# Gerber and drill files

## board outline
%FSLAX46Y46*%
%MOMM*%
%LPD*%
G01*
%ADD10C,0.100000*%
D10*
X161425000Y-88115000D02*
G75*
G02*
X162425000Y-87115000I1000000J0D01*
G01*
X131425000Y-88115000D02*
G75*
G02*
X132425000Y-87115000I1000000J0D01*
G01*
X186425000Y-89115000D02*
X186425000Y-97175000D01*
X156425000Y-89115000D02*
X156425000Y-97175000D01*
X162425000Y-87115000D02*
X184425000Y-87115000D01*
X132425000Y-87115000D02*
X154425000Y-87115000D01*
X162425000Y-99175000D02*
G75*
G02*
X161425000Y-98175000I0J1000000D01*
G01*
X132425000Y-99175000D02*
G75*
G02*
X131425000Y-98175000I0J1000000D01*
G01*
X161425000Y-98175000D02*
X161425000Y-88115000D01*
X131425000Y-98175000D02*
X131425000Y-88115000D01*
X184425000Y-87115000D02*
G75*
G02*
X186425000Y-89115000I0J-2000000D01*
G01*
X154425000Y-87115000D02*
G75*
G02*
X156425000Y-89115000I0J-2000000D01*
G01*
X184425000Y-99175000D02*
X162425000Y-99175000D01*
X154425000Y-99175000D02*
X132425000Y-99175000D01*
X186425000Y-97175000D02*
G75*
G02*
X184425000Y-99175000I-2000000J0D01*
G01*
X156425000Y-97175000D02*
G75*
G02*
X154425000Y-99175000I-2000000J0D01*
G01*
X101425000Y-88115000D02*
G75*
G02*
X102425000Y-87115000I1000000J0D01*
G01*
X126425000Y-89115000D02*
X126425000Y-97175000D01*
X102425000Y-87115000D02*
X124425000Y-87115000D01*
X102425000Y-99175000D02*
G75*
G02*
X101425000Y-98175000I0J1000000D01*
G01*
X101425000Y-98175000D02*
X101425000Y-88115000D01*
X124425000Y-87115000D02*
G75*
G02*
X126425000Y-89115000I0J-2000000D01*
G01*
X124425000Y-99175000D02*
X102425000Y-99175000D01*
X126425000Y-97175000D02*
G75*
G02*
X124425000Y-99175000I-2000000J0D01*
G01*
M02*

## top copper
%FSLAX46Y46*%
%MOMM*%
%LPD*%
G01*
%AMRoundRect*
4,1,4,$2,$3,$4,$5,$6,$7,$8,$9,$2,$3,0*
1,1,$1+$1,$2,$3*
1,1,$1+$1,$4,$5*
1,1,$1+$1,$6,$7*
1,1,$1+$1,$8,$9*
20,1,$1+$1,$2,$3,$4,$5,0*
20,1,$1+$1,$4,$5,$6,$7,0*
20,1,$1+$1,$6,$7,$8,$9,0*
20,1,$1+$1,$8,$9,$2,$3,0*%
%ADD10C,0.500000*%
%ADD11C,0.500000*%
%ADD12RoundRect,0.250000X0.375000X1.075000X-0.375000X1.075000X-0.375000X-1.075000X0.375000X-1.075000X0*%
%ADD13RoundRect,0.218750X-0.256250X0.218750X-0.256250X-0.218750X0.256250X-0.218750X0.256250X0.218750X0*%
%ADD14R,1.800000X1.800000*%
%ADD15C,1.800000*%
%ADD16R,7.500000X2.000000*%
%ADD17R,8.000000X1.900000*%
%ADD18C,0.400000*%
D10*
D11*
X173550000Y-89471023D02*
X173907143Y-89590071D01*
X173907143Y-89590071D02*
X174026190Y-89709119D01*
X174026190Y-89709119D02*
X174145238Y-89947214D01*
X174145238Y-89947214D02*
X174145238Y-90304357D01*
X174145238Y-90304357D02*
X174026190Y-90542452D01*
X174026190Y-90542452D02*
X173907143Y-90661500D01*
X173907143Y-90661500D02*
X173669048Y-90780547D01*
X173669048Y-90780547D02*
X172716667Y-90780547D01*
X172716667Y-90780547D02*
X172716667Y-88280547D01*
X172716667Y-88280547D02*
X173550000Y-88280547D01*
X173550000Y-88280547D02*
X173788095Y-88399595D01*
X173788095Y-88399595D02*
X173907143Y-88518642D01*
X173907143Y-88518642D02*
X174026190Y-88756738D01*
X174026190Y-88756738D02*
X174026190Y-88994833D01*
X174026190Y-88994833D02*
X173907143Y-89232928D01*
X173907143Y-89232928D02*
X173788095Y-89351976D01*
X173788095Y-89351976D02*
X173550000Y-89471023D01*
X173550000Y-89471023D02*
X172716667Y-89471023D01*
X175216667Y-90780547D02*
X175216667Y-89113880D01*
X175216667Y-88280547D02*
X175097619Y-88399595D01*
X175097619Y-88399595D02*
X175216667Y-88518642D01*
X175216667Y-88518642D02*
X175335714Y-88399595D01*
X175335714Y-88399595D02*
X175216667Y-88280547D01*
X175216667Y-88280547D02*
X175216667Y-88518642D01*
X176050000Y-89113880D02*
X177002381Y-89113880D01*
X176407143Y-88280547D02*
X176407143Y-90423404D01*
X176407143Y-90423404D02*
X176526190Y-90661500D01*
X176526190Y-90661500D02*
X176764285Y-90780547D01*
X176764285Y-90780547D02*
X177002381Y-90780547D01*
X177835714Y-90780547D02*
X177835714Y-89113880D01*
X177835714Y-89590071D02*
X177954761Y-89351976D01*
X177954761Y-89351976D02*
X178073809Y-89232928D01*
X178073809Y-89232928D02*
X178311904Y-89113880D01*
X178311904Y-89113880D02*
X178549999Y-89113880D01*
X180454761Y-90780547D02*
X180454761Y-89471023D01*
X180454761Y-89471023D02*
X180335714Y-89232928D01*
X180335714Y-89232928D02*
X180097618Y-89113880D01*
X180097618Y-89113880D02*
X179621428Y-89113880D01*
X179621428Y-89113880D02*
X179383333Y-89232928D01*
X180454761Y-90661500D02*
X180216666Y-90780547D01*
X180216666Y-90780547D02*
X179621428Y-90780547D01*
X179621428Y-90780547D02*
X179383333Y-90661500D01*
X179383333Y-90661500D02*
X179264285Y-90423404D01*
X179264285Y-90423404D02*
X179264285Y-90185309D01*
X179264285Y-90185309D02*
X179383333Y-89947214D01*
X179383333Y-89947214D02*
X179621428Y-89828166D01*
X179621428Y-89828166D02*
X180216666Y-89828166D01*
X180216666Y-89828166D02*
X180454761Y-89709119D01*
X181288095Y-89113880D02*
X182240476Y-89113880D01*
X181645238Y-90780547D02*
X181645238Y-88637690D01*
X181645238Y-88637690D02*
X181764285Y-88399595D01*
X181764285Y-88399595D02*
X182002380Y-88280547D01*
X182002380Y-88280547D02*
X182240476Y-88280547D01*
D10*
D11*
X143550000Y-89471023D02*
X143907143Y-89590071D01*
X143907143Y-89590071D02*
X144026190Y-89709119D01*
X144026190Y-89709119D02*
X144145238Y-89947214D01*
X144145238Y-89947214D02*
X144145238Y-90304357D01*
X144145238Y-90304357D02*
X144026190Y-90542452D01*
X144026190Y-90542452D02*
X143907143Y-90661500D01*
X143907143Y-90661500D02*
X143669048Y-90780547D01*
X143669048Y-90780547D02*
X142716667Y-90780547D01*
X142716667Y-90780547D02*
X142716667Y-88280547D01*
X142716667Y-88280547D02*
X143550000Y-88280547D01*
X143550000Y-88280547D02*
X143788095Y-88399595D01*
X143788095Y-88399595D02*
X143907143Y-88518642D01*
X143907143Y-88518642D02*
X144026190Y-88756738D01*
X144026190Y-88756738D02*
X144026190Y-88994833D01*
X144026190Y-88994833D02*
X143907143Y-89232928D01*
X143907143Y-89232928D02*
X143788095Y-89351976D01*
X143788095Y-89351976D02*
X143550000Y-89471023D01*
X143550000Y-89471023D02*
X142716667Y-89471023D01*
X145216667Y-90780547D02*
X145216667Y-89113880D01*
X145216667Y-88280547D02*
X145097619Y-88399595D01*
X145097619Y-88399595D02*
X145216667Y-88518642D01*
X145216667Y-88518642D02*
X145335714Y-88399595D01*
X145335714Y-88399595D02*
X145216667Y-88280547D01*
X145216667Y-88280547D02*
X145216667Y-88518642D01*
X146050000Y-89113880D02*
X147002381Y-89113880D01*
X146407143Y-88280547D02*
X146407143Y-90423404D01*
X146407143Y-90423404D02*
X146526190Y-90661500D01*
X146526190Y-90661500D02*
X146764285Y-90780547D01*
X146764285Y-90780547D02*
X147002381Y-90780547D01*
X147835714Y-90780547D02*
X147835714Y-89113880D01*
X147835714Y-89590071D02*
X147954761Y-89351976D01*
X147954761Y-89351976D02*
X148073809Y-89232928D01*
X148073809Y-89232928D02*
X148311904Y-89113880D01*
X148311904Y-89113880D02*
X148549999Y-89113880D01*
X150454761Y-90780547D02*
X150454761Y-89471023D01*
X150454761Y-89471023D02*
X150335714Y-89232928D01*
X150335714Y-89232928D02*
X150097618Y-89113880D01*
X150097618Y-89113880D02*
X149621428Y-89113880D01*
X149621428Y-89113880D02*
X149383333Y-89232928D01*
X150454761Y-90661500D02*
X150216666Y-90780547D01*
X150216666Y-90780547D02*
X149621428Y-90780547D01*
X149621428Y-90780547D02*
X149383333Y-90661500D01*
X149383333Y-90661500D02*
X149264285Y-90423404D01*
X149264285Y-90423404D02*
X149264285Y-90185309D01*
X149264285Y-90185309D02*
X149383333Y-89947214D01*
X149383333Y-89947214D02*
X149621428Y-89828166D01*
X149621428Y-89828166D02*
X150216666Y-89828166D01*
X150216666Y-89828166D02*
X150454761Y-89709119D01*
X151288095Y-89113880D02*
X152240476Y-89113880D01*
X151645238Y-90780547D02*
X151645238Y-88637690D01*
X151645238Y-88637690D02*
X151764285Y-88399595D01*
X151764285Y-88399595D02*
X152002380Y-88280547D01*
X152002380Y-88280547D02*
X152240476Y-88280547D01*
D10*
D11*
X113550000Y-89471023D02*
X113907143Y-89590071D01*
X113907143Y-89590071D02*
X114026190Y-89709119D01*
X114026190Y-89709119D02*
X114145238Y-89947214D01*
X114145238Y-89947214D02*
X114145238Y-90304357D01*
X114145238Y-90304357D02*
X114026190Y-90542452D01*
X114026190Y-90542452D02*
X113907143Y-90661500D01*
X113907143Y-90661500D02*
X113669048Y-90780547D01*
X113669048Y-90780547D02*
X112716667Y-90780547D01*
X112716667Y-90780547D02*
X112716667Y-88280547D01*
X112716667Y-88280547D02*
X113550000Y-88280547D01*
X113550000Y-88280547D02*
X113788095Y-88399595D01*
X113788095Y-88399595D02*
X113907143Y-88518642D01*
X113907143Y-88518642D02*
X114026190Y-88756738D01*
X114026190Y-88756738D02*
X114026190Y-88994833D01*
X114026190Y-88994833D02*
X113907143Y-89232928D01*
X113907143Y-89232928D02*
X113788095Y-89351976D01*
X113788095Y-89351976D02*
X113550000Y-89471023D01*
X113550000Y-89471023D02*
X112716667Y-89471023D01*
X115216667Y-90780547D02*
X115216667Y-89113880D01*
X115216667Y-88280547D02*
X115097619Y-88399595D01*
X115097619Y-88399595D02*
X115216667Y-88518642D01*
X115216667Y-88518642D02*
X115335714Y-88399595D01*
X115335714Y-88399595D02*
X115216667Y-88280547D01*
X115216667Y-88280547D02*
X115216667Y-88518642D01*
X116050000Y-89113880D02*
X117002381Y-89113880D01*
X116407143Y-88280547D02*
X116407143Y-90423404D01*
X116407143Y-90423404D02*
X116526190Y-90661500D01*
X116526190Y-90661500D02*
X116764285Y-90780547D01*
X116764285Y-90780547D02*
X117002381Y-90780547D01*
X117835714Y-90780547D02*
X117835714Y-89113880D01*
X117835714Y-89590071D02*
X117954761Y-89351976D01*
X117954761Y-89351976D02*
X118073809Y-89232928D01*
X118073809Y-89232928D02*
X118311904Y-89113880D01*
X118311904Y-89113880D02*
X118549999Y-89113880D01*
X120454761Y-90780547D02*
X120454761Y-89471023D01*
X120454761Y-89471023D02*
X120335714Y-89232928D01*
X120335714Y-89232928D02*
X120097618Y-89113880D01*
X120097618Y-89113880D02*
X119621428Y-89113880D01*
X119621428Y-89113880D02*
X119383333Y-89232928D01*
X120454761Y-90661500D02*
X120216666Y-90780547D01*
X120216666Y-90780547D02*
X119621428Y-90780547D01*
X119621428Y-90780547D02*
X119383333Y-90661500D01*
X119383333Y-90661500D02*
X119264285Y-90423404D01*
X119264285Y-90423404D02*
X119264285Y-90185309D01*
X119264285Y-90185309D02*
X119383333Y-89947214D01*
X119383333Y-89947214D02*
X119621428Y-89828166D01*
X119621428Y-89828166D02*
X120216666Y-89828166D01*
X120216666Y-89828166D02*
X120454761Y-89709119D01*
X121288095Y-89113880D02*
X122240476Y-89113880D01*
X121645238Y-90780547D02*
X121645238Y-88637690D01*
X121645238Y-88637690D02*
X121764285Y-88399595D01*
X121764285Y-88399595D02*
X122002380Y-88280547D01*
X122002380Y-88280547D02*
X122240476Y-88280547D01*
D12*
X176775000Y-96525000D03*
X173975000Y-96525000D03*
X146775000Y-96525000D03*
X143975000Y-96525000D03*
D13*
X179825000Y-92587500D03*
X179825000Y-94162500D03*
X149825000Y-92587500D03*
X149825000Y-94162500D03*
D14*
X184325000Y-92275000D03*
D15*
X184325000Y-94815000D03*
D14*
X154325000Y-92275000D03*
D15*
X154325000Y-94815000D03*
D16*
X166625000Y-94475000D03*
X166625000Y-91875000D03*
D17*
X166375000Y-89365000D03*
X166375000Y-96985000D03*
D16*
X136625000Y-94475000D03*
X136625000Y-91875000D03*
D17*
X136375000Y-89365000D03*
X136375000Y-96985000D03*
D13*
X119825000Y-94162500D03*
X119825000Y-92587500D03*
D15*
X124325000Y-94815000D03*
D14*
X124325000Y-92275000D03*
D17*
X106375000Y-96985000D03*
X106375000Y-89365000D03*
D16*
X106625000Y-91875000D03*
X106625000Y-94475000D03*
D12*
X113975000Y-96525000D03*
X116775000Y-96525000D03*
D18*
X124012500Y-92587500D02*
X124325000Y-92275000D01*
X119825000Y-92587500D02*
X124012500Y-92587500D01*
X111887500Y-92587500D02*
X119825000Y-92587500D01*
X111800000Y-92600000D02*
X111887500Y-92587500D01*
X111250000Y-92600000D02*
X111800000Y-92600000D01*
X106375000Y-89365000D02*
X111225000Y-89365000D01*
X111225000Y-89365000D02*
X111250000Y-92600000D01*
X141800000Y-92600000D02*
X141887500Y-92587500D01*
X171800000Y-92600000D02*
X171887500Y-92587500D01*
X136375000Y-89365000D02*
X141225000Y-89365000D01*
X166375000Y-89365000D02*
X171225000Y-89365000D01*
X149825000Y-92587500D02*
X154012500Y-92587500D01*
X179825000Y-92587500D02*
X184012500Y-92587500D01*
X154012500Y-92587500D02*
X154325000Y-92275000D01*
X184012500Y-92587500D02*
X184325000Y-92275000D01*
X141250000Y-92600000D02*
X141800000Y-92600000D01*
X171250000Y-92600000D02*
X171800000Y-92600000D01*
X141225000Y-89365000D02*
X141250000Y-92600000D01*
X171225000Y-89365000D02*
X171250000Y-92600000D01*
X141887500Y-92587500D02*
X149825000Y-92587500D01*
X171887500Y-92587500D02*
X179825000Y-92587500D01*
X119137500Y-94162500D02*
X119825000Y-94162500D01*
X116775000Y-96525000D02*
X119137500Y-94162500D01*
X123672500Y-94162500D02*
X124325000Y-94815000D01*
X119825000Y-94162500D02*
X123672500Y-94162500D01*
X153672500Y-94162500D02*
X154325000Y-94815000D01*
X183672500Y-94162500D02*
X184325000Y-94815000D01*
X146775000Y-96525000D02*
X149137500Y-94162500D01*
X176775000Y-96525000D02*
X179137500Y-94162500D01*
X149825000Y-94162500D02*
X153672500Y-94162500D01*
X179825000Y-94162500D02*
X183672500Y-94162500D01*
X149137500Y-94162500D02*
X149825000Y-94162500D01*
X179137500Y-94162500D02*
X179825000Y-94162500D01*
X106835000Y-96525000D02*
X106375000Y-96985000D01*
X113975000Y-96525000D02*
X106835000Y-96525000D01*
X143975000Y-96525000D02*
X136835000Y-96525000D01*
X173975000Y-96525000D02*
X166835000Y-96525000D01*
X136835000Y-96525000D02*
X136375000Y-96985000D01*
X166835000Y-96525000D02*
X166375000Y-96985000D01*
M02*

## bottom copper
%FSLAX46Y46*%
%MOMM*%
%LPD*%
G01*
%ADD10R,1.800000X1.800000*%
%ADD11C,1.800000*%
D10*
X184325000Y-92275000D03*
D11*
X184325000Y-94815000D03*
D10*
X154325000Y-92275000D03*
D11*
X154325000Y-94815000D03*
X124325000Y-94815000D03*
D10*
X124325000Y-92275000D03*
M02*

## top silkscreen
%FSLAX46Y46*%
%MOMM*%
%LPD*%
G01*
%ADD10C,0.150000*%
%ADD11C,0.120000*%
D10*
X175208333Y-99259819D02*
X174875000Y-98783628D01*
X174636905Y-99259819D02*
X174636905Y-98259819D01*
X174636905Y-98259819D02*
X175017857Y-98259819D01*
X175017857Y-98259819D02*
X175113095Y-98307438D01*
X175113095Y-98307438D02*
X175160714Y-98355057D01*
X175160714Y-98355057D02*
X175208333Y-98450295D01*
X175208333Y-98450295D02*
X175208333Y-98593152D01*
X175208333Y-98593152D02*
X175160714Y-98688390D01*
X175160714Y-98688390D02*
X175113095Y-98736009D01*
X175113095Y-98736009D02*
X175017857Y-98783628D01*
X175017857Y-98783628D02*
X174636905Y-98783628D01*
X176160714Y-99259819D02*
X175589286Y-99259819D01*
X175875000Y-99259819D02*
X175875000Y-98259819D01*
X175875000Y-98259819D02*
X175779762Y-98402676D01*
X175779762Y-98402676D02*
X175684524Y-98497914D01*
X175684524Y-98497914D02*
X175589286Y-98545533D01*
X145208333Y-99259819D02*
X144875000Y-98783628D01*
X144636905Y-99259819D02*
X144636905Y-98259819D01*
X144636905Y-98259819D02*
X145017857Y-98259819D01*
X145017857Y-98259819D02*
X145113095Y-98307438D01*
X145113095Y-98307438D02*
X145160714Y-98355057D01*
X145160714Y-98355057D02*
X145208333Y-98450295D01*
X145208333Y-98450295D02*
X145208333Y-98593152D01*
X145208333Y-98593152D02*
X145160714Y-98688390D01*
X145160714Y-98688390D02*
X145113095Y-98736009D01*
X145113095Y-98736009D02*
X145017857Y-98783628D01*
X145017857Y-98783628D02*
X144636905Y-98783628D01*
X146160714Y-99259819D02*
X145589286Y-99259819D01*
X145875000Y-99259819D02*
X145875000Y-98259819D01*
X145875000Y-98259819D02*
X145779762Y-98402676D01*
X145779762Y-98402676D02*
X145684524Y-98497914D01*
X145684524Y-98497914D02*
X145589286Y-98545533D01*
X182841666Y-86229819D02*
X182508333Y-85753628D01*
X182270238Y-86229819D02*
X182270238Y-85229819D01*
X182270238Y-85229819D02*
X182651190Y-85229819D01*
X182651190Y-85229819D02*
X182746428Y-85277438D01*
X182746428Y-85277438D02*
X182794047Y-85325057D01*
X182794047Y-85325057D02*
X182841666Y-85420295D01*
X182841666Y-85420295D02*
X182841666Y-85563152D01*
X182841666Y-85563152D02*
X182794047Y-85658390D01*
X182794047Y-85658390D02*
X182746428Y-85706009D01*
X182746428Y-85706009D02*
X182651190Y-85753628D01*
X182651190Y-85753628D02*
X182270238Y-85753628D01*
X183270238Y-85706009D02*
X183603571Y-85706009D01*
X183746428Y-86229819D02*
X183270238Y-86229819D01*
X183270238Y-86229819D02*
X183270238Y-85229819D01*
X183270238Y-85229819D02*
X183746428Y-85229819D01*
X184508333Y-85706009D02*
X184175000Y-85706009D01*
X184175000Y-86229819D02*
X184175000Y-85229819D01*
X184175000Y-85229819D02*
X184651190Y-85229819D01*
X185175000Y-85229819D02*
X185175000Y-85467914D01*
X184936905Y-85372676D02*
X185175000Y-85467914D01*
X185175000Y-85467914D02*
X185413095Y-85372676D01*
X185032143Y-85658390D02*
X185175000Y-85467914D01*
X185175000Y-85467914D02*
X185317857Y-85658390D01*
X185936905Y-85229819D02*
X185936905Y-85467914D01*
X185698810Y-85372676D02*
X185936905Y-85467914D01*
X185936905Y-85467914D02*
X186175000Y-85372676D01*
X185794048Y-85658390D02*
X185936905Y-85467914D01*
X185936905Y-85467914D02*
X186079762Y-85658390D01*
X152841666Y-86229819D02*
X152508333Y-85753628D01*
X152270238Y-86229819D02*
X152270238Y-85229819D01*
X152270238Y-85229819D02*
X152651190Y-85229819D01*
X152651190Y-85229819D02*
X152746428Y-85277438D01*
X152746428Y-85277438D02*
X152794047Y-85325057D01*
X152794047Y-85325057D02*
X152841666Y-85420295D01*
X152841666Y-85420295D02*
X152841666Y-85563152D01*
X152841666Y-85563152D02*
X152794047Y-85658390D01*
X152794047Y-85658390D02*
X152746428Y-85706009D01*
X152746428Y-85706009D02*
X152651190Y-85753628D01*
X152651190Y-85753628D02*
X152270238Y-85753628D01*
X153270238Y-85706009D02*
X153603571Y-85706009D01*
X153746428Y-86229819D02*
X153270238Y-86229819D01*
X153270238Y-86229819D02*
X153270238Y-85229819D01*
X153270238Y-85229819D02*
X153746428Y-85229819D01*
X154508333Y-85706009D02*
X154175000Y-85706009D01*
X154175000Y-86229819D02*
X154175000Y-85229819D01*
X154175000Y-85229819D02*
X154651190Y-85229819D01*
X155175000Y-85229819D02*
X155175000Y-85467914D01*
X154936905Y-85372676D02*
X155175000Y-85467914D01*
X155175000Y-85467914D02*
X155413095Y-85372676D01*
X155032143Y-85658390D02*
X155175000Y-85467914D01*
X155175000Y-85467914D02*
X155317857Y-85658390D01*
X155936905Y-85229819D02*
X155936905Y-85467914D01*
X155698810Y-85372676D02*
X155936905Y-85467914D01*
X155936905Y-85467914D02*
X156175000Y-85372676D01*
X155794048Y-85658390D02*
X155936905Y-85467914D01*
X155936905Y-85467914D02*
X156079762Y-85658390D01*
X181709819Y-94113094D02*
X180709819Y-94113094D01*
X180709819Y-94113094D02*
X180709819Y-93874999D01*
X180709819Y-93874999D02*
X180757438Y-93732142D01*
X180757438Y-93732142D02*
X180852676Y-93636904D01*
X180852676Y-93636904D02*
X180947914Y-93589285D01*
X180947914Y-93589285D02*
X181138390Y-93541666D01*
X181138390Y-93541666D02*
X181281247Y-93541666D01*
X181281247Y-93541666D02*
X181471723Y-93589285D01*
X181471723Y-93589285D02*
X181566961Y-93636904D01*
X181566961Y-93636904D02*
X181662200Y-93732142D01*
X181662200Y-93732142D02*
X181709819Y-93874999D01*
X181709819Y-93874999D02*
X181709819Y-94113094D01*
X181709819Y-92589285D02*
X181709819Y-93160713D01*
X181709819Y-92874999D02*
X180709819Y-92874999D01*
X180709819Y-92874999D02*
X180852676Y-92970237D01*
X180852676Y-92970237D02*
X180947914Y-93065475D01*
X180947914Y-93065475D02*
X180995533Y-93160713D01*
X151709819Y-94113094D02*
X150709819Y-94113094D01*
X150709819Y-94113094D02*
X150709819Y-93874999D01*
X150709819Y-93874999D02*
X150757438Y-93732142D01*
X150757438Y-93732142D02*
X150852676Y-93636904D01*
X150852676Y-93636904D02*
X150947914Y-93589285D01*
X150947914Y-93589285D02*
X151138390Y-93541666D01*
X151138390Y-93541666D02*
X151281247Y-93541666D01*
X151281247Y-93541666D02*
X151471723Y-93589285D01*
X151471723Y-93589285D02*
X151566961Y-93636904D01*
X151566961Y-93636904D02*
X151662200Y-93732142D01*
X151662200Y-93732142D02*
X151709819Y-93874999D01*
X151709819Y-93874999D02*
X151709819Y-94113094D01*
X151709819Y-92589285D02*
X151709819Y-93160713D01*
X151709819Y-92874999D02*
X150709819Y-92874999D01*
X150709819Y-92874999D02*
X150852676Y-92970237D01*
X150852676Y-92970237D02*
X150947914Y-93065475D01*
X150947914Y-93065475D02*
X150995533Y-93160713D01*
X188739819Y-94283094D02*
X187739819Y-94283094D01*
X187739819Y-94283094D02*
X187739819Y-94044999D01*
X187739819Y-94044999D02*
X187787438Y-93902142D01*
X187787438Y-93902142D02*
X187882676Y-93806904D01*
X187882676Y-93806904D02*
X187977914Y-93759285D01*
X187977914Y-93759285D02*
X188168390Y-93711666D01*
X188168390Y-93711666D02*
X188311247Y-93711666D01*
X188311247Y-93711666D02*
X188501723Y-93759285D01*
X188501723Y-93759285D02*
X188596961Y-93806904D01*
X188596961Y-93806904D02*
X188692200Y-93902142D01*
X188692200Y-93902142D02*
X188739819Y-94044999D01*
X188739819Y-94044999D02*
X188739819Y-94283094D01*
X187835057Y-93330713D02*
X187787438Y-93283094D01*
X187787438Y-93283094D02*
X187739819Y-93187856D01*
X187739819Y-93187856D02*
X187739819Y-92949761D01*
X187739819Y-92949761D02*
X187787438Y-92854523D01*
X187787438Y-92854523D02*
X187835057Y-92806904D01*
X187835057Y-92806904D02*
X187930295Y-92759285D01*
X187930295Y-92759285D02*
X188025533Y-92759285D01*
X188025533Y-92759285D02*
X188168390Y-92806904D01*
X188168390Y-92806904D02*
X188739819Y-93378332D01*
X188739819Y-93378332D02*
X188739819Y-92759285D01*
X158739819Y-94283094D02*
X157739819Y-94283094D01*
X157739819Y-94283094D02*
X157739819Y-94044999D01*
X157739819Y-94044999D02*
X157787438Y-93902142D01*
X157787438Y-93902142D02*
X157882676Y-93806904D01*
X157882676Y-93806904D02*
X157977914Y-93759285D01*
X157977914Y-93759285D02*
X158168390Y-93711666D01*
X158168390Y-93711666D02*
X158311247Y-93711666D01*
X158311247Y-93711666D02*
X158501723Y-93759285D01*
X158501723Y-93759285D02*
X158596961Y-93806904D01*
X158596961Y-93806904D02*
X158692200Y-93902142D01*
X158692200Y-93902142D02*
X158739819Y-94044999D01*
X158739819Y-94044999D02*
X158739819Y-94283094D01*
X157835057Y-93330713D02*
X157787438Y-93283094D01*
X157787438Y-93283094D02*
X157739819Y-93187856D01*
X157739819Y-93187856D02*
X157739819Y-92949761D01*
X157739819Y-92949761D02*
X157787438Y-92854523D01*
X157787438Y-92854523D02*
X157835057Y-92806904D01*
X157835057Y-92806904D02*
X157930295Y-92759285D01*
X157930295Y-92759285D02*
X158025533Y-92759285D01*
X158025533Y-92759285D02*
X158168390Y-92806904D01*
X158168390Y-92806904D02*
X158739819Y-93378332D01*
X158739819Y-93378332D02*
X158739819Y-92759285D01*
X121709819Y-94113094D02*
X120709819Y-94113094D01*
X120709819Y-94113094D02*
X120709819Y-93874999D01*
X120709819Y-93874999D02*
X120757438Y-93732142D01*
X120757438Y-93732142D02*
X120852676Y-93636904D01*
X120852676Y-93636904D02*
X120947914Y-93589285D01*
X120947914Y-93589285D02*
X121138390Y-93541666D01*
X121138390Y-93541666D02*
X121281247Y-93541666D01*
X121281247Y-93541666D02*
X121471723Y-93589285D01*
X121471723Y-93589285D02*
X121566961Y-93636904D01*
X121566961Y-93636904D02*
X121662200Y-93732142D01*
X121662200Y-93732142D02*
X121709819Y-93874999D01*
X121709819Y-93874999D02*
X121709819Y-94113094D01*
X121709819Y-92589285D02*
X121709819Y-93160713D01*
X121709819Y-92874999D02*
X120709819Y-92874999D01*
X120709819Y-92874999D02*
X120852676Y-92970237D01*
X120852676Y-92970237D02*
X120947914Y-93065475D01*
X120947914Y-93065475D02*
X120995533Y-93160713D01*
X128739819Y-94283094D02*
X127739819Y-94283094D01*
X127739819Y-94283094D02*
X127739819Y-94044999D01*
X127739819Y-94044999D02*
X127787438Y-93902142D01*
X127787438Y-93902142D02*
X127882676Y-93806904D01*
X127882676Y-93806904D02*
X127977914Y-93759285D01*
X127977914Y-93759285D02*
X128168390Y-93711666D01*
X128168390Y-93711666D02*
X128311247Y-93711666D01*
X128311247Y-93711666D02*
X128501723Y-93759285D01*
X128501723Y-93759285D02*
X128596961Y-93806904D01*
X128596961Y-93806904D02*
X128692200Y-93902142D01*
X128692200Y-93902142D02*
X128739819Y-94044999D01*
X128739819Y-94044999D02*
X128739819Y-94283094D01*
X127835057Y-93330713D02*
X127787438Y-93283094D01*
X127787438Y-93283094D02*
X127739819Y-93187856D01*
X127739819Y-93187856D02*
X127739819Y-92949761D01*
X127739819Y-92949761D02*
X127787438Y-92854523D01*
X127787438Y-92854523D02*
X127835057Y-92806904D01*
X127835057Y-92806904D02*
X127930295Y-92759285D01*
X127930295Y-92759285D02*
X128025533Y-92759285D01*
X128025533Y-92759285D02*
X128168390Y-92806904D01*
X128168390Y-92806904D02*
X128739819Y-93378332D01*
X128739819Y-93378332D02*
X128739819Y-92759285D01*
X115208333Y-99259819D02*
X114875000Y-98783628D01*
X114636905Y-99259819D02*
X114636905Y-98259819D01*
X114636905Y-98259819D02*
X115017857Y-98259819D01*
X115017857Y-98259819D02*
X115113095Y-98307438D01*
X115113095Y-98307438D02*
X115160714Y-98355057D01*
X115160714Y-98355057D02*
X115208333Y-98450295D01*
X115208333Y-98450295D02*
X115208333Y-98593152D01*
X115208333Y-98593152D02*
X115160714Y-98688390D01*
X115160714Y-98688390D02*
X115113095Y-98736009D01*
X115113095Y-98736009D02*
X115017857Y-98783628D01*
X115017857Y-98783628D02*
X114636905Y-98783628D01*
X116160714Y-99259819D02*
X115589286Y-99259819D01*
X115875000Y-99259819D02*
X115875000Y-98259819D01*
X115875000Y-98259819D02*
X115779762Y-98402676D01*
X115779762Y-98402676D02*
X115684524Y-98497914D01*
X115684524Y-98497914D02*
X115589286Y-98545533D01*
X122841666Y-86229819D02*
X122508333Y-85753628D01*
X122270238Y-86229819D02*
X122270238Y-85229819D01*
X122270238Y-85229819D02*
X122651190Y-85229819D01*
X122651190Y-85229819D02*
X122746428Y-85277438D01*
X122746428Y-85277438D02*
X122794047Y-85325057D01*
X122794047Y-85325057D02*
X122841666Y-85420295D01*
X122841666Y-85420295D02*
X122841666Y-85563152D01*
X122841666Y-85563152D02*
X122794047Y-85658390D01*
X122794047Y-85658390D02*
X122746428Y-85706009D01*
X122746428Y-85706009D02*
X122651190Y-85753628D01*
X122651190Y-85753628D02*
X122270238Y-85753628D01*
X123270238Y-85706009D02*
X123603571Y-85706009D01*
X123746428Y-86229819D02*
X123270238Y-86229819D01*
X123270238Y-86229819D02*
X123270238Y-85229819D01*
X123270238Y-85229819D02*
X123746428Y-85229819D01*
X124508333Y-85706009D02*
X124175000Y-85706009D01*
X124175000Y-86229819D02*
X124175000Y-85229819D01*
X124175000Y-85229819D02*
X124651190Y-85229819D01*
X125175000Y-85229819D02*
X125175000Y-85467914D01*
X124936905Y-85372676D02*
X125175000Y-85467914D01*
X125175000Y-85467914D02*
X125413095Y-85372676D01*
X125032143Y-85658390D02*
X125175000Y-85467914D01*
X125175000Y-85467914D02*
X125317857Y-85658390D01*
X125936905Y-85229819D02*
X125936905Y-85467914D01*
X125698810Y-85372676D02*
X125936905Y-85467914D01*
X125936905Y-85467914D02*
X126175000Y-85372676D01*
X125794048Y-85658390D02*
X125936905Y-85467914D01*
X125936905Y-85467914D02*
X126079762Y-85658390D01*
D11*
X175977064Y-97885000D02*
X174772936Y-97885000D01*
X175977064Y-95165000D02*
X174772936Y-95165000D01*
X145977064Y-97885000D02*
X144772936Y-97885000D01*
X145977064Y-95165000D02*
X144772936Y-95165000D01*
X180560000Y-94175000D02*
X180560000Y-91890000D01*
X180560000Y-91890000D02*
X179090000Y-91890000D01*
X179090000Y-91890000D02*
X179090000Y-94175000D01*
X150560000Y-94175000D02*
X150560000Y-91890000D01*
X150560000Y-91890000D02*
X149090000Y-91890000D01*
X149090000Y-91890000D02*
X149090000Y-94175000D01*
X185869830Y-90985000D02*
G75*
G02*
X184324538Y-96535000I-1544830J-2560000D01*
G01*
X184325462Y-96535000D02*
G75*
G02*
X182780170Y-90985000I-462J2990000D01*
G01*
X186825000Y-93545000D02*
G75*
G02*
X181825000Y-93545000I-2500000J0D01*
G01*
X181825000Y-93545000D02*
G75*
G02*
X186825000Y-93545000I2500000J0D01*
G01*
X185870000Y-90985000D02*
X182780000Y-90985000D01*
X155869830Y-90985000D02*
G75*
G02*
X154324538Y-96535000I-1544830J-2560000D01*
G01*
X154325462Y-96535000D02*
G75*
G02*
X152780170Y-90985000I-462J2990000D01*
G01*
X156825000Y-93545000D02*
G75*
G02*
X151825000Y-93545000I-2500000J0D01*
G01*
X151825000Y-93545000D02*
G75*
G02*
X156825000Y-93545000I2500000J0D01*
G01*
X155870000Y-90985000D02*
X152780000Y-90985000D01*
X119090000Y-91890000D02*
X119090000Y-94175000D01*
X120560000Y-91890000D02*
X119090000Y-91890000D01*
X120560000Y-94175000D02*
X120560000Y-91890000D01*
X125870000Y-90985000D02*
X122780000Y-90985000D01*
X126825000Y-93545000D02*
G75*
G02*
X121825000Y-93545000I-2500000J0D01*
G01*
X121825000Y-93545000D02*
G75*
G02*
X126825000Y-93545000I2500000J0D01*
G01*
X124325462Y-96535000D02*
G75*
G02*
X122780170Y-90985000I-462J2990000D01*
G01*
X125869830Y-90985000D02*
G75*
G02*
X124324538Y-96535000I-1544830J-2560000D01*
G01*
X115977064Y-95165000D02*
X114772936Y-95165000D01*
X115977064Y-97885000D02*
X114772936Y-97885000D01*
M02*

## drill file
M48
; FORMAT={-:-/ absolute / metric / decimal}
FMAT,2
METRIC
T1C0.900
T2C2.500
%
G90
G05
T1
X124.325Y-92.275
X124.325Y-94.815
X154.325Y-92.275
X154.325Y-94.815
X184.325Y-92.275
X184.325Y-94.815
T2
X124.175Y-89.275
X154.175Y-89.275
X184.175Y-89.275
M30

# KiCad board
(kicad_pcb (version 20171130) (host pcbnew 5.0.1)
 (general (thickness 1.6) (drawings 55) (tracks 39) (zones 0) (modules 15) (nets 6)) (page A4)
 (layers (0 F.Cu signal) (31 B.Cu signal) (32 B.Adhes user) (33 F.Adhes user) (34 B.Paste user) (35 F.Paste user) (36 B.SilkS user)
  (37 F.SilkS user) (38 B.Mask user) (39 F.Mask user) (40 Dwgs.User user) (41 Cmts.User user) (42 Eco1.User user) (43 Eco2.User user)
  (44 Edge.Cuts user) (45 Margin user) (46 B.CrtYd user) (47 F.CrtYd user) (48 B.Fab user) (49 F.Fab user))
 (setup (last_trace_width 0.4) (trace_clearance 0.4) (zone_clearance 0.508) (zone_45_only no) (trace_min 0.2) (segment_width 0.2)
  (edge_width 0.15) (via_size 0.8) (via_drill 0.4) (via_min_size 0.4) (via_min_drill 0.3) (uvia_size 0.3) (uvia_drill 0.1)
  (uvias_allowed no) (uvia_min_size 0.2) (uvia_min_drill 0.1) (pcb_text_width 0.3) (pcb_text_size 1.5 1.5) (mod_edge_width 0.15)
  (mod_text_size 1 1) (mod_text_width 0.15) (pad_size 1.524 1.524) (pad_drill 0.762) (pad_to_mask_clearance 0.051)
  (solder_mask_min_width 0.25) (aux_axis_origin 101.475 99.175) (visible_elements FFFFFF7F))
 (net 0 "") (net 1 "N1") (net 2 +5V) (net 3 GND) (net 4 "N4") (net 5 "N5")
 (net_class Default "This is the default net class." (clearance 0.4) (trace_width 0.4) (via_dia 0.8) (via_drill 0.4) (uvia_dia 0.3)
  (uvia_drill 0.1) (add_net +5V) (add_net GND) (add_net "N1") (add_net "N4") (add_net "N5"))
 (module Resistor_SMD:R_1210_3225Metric (layer F.Cu) (at 175.375 96.525 180)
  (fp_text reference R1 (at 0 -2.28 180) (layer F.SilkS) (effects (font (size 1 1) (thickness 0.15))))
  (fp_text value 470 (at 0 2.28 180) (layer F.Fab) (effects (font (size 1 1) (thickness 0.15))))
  (fp_line (start -0.602064 -1.36) (end 0.602064 -1.36) (layer F.SilkS) (width 0.12))
  (fp_line (start -0.602064 1.36) (end 0.602064 1.36) (layer F.SilkS) (width 0.12))
  (pad 1 smd roundrect (at -1.4 0 180) (size 1.25 2.65) (layers F.Cu F.Paste F.Mask) (roundrect_rratio 0.2) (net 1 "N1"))
  (pad 2 smd roundrect (at 1.4 0 180) (size 1.25 2.65) (layers F.Cu F.Paste F.Mask) (roundrect_rratio 0.2) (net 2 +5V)))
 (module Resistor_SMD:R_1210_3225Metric (layer F.Cu) (at 145.375 96.525 180)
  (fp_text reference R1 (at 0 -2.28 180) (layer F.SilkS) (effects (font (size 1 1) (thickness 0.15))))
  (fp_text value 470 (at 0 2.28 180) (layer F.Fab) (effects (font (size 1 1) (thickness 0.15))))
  (fp_line (start -0.602064 -1.36) (end 0.602064 -1.36) (layer F.SilkS) (width 0.12))
  (fp_line (start -0.602064 1.36) (end 0.602064 1.36) (layer F.SilkS) (width 0.12))
  (pad 1 smd roundrect (at -1.4 0 180) (size 1.25 2.65) (layers F.Cu F.Paste F.Mask) (roundrect_rratio 0.2) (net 1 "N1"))
  (pad 2 smd roundrect (at 1.4 0 180) (size 1.25 2.65) (layers F.Cu F.Paste F.Mask) (roundrect_rratio 0.2) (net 2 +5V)))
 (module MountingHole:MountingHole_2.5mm (layer F.Cu) (at 184.175 89.275)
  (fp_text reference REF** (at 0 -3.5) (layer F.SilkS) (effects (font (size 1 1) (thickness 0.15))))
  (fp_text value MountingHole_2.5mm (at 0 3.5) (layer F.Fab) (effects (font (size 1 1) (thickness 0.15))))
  (pad 1 np_thru_hole circle (at 0 0) (size 2.5 2.5) (drill 2.5) (layers *.Cu *.Mask)))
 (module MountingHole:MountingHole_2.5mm (layer F.Cu) (at 154.175 89.275)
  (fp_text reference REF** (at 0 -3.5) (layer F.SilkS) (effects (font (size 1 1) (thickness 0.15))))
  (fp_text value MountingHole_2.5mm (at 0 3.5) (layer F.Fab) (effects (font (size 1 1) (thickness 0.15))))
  (pad 1 np_thru_hole circle (at 0 0) (size 2.5 2.5) (drill 2.5) (layers *.Cu *.Mask)))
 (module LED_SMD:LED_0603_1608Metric (layer F.Cu) (at 179.825 93.375 270)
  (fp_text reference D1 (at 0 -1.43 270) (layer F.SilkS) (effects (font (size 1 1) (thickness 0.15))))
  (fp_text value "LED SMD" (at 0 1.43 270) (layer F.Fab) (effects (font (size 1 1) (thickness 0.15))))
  (fp_line (start 0.8 -0.735) (end -1.485 -0.735) (layer F.SilkS) (width 0.12))
  (fp_line (start -1.485 -0.735) (end -1.485 0.735) (layer F.SilkS) (width 0.12))
  (fp_line (start -1.485 0.735) (end 0.8 0.735) (layer F.SilkS) (width 0.12))
  (pad 1 smd roundrect (at -0.7875 0 270) (size 0.875 0.95) (layers F.Cu F.Paste F.Mask) (roundrect_rratio 0.25) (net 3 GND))
  (pad 2 smd roundrect (at 0.7875 0 270) (size 0.875 0.95) (layers F.Cu F.Paste F.Mask) (roundrect_rratio 0.25) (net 1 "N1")))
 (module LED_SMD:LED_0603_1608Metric (layer F.Cu) (at 149.825 93.375 270)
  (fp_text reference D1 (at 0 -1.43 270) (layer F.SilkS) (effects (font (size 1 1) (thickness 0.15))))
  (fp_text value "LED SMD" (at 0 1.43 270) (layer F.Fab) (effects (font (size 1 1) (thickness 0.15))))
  (fp_line (start 0.8 -0.735) (end -1.485 -0.735) (layer F.SilkS) (width 0.12))
  (fp_line (start -1.485 -0.735) (end -1.485 0.735) (layer F.SilkS) (width 0.12))
  (fp_line (start -1.485 0.735) (end 0.8 0.735) (layer F.SilkS) (width 0.12))
  (pad 1 smd roundrect (at -0.7875 0 270) (size 0.875 0.95) (layers F.Cu F.Paste F.Mask) (roundrect_rratio 0.25) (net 3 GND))
  (pad 2 smd roundrect (at 0.7875 0 270) (size 0.875 0.95) (layers F.Cu F.Paste F.Mask) (roundrect_rratio 0.25) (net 1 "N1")))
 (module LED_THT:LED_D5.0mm (layer F.Cu) (at 184.325 92.275 270)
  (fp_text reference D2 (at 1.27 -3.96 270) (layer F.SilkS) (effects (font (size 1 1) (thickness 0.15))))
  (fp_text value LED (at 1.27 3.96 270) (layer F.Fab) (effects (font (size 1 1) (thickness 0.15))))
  (fp_arc (start 1.27 0) (end -1.29 -1.54483) (angle 148.9) (layer F.SilkS) (width 0.12))
  (fp_arc (start 1.27 0) (end -1.29 1.54483) (angle -148.9) (layer F.SilkS) (width 0.12))
  (fp_circle (center 1.27 0) (end 3.77 0) (layer F.SilkS) (width 0.12))
  (fp_line (start -1.29 -1.545) (end -1.29 1.545) (layer F.SilkS) (width 0.12))
  (pad 1 thru_hole rect (at 0 0 270) (size 1.8 1.8) (drill 0.9) (layers *.Cu *.Mask) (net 3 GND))
  (pad 2 thru_hole circle (at 2.54 0 270) (size 1.8 1.8) (drill 0.9) (layers *.Cu *.Mask) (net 1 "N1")))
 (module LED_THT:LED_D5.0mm (layer F.Cu) (at 154.325 92.275 270)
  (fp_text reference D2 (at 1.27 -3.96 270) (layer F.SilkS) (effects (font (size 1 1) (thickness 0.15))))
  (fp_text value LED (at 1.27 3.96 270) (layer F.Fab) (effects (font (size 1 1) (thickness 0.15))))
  (fp_arc (start 1.27 0) (end -1.29 -1.54483) (angle 148.9) (layer F.SilkS) (width 0.12))
  (fp_arc (start 1.27 0) (end -1.29 1.54483) (angle -148.9) (layer F.SilkS) (width 0.12))
  (fp_circle (center 1.27 0) (end 3.77 0) (layer F.SilkS) (width 0.12))
  (fp_line (start -1.29 -1.545) (end -1.29 1.545) (layer F.SilkS) (width 0.12))
  (pad 1 thru_hole rect (at 0 0 270) (size 1.8 1.8) (drill 0.9) (layers *.Cu *.Mask) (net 3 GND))
  (pad 2 thru_hole circle (at 2.54 0 270) (size 1.8 1.8) (drill 0.9) (layers *.Cu *.Mask) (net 1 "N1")))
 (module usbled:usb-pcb (layer F.Cu) (at 161.475 93.175 270)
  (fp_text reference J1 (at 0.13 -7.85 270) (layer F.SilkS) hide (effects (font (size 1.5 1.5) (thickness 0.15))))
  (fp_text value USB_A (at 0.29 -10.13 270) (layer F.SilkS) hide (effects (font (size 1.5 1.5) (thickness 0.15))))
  (pad 2 connect rect (at 1.3 -5.15 270) (size 2 7.5) (layers F.Cu F.Mask) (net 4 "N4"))
  (pad 3 connect rect (at -1.3 -5.15 270) (size 2 7.5) (layers F.Cu F.Mask) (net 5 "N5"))
  (pad 4 connect rect (at -3.81 -4.9 270) (size 1.9 8) (layers F.Cu F.Mask) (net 3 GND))
  (pad 1 connect rect (at 3.81 -4.9 270) (size 1.9 8) (layers F.Cu F.Mask) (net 2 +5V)))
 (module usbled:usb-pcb (layer F.Cu) (at 131.475 93.175 270)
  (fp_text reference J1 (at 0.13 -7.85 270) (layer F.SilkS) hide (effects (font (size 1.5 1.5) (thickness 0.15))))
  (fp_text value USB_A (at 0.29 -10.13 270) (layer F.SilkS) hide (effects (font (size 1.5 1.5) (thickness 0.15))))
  (pad 2 connect rect (at 1.3 -5.15 270) (size 2 7.5) (layers F.Cu F.Mask) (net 4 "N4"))
  (pad 3 connect rect (at -1.3 -5.15 270) (size 2 7.5) (layers F.Cu F.Mask) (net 5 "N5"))
  (pad 4 connect rect (at -3.81 -4.9 270) (size 1.9 8) (layers F.Cu F.Mask) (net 3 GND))
  (pad 1 connect rect (at 3.81 -4.9 270) (size 1.9 8) (layers F.Cu F.Mask) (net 2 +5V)))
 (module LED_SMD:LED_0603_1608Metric (layer F.Cu) (at 119.825 93.375 270)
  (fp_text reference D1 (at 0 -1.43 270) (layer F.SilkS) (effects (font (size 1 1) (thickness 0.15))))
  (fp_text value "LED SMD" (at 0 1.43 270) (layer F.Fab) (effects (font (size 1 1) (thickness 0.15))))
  (fp_line (start -1.485 0.735) (end 0.8 0.735) (layer F.SilkS) (width 0.12))
  (fp_line (start -1.485 -0.735) (end -1.485 0.735) (layer F.SilkS) (width 0.12))
  (fp_line (start 0.8 -0.735) (end -1.485 -0.735) (layer F.SilkS) (width 0.12))
  (pad 2 smd roundrect (at 0.7875 0 270) (size 0.875 0.95) (layers F.Cu F.Paste F.Mask) (roundrect_rratio 0.25) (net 1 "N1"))
  (pad 1 smd roundrect (at -0.7875 0 270) (size 0.875 0.95) (layers F.Cu F.Paste F.Mask) (roundrect_rratio 0.25) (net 3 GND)))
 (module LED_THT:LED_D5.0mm (layer F.Cu) (at 124.325 92.275 270)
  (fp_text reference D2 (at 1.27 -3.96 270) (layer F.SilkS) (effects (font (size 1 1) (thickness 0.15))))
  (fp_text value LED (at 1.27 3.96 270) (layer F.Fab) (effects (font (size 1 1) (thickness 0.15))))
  (fp_line (start -1.29 -1.545) (end -1.29 1.545) (layer F.SilkS) (width 0.12))
  (fp_circle (center 1.27 0) (end 3.77 0) (layer F.SilkS) (width 0.12))
  (fp_arc (start 1.27 0) (end -1.29 1.54483) (angle -148.9) (layer F.SilkS) (width 0.12))
  (fp_arc (start 1.27 0) (end -1.29 -1.54483) (angle 148.9) (layer F.SilkS) (width 0.12))
  (pad 2 thru_hole circle (at 2.54 0 270) (size 1.8 1.8) (drill 0.9) (layers *.Cu *.Mask) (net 1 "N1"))
  (pad 1 thru_hole rect (at 0 0 270) (size 1.8 1.8) (drill 0.9) (layers *.Cu *.Mask) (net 3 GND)))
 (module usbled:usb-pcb (layer F.Cu) (at 101.475 93.175 270)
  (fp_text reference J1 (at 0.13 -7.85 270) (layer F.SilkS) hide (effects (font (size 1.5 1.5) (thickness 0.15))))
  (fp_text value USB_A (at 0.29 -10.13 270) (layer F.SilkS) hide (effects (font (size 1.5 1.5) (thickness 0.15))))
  (pad 1 connect rect (at 3.81 -4.9 270) (size 1.9 8) (layers F.Cu F.Mask) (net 2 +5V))
  (pad 4 connect rect (at -3.81 -4.9 270) (size 1.9 8) (layers F.Cu F.Mask) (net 3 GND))
  (pad 3 connect rect (at -1.3 -5.15 270) (size 2 7.5) (layers F.Cu F.Mask) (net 5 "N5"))
  (pad 2 connect rect (at 1.3 -5.15 270) (size 2 7.5) (layers F.Cu F.Mask) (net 4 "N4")))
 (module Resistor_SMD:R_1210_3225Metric (layer F.Cu) (at 115.375 96.525 180)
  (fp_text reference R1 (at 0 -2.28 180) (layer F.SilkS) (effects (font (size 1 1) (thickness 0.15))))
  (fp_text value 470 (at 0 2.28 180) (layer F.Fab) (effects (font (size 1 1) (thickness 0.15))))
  (fp_line (start -0.602064 1.36) (end 0.602064 1.36) (layer F.SilkS) (width 0.12))
  (fp_line (start -0.602064 -1.36) (end 0.602064 -1.36) (layer F.SilkS) (width 0.12))
  (pad 2 smd roundrect (at 1.4 0 180) (size 1.25 2.65) (layers F.Cu F.Paste F.Mask) (roundrect_rratio 0.2) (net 2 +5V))
  (pad 1 smd roundrect (at -1.4 0 180) (size 1.25 2.65) (layers F.Cu F.Paste F.Mask) (roundrect_rratio 0.2) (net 1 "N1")))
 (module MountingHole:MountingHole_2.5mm (layer F.Cu) (at 124.175 89.275)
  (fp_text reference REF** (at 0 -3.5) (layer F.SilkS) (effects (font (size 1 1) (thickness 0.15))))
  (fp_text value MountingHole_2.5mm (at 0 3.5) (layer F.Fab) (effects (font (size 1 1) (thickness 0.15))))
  (pad 1 np_thru_hole circle (at 0 0) (size 2.5 2.5) (drill 2.5) (layers *.Cu *.Mask)))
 (gr_arc (start 162.425 88.115) (end 162.425 87.115) (angle -90) (layer Edge.Cuts) (width 0.1))
 (gr_arc (start 132.425 88.115) (end 132.425 87.115) (angle -90) (layer Edge.Cuts) (width 0.1))
 (gr_line (start 186.425 89.115) (end 186.425 97.175) (layer Edge.Cuts) (width 0.1))
 (gr_line (start 156.425 89.115) (end 156.425 97.175) (layer Edge.Cuts) (width 0.1))
 (gr_line (start 162.425 87.115) (end 184.425 87.115) (layer Edge.Cuts) (width 0.1))
 (gr_line (start 132.425 87.115) (end 154.425 87.115) (layer Edge.Cuts) (width 0.1))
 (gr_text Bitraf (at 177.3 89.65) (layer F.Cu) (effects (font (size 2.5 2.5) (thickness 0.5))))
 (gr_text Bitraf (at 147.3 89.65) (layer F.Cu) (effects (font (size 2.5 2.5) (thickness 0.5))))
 (gr_arc (start 162.425 98.175) (end 161.425 98.175) (angle -90) (layer Edge.Cuts) (width 0.1))
 (gr_arc (start 132.425 98.175) (end 131.425 98.175) (angle -90) (layer Edge.Cuts) (width 0.1))
 (gr_line (start 161.425 98.175) (end 161.425 88.115) (layer Edge.Cuts) (width 0.1))
 (gr_line (start 131.425 98.175) (end 131.425 88.115) (layer Edge.Cuts) (width 0.1))
 (gr_arc (start 184.425 89.115) (end 186.425 89.115) (angle -90) (layer Edge.Cuts) (width 0.1))
 (gr_arc (start 154.425 89.115) (end 156.425 89.115) (angle -90) (layer Edge.Cuts) (width 0.1))
 (gr_line (start 184.425 99.175) (end 162.425 99.175) (layer Edge.Cuts) (width 0.1))
 (gr_line (start 154.425 99.175) (end 132.425 99.175) (layer Edge.Cuts) (width 0.1))
 (gr_arc (start 184.425 97.175) (end 184.425 99.175) (angle -90) (layer Edge.Cuts) (width 0.1))
 (gr_arc (start 154.425 97.175) (end 154.425 99.175) (angle -90) (layer Edge.Cuts) (width 0.1))
 (gr_arc (start 102.425 88.115) (end 102.425 87.115) (angle -90) (layer Edge.Cuts) (width 0.1))
 (gr_line (start 126.425 89.115) (end 126.425 97.175) (layer Edge.Cuts) (width 0.1))
 (gr_line (start 102.425 87.115) (end 124.425 87.115) (layer Edge.Cuts) (width 0.1))
 (gr_arc (start 102.425 98.175) (end 101.425 98.175) (angle -90) (layer Edge.Cuts) (width 0.1))
 (gr_line (start 101.425 98.175) (end 101.425 88.115) (layer Edge.Cuts) (width 0.1))
 (gr_arc (start 124.425 89.115) (end 126.425 89.115) (angle -90) (layer Edge.Cuts) (width 0.1))
 (gr_line (start 124.425 99.175) (end 102.425 99.175) (layer Edge.Cuts) (width 0.1))
 (gr_arc (start 124.425 97.175) (end 124.425 99.175) (angle -90) (layer Edge.Cuts) (width 0.1))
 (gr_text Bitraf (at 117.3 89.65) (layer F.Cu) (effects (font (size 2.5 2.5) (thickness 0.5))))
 (segment (start 124.0125 92.5875) (end 124.325 92.275) (width 0.4) (layer F.Cu) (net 3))
 (segment (start 119.825 92.5875) (end 124.0125 92.5875) (width 0.4) (layer F.Cu) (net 3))
 (segment (start 111.8875 92.5875) (end 119.825 92.5875) (width 0.4) (layer F.Cu) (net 3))
 (segment (start 111.8 92.6) (end 111.8875 92.5875) (width 0.4) (layer F.Cu) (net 3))
 (segment (start 111.25 92.6) (end 111.8 92.6) (width 0.4) (layer F.Cu) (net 3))
 (segment (start 106.375 89.365) (end 111.225 89.365) (width 0.4) (layer F.Cu) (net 3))
 (segment (start 111.225 89.365) (end 111.25 92.6) (width 0.4) (layer F.Cu) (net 3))
 (segment (start 141.8 92.6) (end 141.8875 92.5875) (width 0.4) (layer F.Cu) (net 3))
 (segment (start 171.8 92.6) (end 171.8875 92.5875) (width 0.4) (layer F.Cu) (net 3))
 (segment (start 136.375 89.365) (end 141.225 89.365) (width 0.4) (layer F.Cu) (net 3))
 (segment (start 166.375 89.365) (end 171.225 89.365) (width 0.4) (layer F.Cu) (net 3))
 (segment (start 149.825 92.5875) (end 154.0125 92.5875) (width 0.4) (layer F.Cu) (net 3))
 (segment (start 179.825 92.5875) (end 184.0125 92.5875) (width 0.4) (layer F.Cu) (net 3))
 (segment (start 154.0125 92.5875) (end 154.325 92.275) (width 0.4) (layer F.Cu) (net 3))
 (segment (start 184.0125 92.5875) (end 184.325 92.275) (width 0.4) (layer F.Cu) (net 3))
 (segment (start 141.25 92.6) (end 141.8 92.6) (width 0.4) (layer F.Cu) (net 3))
 (segment (start 171.25 92.6) (end 171.8 92.6) (width 0.4) (layer F.Cu) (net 3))
 (segment (start 141.225 89.365) (end 141.25 92.6) (width 0.4) (layer F.Cu) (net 3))
 (segment (start 171.225 89.365) (end 171.25 92.6) (width 0.4) (layer F.Cu) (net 3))
 (segment (start 141.8875 92.5875) (end 149.825 92.5875) (width 0.4) (layer F.Cu) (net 3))
 (segment (start 171.8875 92.5875) (end 179.825 92.5875) (width 0.4) (layer F.Cu) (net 3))
 (segment (start 119.1375 94.1625) (end 119.825 94.1625) (width 0.4) (layer F.Cu) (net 1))
 (segment (start 116.775 96.525) (end 119.1375 94.1625) (width 0.4) (layer F.Cu) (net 1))
 (segment (start 123.6725 94.1625) (end 124.325 94.815) (width 0.4) (layer F.Cu) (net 1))
 (segment (start 119.825 94.1625) (end 123.6725 94.1625) (width 0.4) (layer F.Cu) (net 1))
 (segment (start 153.6725 94.1625) (end 154.325 94.815) (width 0.4) (layer F.Cu) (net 1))
 (segment (start 183.6725 94.1625) (end 184.325 94.815) (width 0.4) (layer F.Cu) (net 1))
 (segment (start 146.775 96.525) (end 149.1375 94.1625) (width 0.4) (layer F.Cu) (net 1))
 (segment (start 176.775 96.525) (end 179.1375 94.1625) (width 0.4) (layer F.Cu) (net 1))
 (segment (start 149.825 94.1625) (end 153.6725 94.1625) (width 0.4) (layer F.Cu) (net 1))
 (segment (start 179.825 94.1625) (end 183.6725 94.1625) (width 0.4) (layer F.Cu) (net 1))
 (segment (start 149.1375 94.1625) (end 149.825 94.1625) (width 0.4) (layer F.Cu) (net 1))
 (segment (start 179.1375 94.1625) (end 179.825 94.1625) (width 0.4) (layer F.Cu) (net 1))
 (segment (start 106.835 96.525) (end 106.375 96.985) (width 0.4) (layer F.Cu) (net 2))
 (segment (start 113.975 96.525) (end 106.835 96.525) (width 0.4) (layer F.Cu) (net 2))
 (segment (start 143.975 96.525) (end 136.835 96.525) (width 0.4) (layer F.Cu) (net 2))
 (segment (start 173.975 96.525) (end 166.835 96.525) (width 0.4) (layer F.Cu) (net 2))
 (segment (start 136.835 96.525) (end 136.375 96.985) (width 0.4) (layer F.Cu) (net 2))
 (segment (start 166.835 96.525) (end 166.375 96.985) (width 0.4) (layer F.Cu) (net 2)))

